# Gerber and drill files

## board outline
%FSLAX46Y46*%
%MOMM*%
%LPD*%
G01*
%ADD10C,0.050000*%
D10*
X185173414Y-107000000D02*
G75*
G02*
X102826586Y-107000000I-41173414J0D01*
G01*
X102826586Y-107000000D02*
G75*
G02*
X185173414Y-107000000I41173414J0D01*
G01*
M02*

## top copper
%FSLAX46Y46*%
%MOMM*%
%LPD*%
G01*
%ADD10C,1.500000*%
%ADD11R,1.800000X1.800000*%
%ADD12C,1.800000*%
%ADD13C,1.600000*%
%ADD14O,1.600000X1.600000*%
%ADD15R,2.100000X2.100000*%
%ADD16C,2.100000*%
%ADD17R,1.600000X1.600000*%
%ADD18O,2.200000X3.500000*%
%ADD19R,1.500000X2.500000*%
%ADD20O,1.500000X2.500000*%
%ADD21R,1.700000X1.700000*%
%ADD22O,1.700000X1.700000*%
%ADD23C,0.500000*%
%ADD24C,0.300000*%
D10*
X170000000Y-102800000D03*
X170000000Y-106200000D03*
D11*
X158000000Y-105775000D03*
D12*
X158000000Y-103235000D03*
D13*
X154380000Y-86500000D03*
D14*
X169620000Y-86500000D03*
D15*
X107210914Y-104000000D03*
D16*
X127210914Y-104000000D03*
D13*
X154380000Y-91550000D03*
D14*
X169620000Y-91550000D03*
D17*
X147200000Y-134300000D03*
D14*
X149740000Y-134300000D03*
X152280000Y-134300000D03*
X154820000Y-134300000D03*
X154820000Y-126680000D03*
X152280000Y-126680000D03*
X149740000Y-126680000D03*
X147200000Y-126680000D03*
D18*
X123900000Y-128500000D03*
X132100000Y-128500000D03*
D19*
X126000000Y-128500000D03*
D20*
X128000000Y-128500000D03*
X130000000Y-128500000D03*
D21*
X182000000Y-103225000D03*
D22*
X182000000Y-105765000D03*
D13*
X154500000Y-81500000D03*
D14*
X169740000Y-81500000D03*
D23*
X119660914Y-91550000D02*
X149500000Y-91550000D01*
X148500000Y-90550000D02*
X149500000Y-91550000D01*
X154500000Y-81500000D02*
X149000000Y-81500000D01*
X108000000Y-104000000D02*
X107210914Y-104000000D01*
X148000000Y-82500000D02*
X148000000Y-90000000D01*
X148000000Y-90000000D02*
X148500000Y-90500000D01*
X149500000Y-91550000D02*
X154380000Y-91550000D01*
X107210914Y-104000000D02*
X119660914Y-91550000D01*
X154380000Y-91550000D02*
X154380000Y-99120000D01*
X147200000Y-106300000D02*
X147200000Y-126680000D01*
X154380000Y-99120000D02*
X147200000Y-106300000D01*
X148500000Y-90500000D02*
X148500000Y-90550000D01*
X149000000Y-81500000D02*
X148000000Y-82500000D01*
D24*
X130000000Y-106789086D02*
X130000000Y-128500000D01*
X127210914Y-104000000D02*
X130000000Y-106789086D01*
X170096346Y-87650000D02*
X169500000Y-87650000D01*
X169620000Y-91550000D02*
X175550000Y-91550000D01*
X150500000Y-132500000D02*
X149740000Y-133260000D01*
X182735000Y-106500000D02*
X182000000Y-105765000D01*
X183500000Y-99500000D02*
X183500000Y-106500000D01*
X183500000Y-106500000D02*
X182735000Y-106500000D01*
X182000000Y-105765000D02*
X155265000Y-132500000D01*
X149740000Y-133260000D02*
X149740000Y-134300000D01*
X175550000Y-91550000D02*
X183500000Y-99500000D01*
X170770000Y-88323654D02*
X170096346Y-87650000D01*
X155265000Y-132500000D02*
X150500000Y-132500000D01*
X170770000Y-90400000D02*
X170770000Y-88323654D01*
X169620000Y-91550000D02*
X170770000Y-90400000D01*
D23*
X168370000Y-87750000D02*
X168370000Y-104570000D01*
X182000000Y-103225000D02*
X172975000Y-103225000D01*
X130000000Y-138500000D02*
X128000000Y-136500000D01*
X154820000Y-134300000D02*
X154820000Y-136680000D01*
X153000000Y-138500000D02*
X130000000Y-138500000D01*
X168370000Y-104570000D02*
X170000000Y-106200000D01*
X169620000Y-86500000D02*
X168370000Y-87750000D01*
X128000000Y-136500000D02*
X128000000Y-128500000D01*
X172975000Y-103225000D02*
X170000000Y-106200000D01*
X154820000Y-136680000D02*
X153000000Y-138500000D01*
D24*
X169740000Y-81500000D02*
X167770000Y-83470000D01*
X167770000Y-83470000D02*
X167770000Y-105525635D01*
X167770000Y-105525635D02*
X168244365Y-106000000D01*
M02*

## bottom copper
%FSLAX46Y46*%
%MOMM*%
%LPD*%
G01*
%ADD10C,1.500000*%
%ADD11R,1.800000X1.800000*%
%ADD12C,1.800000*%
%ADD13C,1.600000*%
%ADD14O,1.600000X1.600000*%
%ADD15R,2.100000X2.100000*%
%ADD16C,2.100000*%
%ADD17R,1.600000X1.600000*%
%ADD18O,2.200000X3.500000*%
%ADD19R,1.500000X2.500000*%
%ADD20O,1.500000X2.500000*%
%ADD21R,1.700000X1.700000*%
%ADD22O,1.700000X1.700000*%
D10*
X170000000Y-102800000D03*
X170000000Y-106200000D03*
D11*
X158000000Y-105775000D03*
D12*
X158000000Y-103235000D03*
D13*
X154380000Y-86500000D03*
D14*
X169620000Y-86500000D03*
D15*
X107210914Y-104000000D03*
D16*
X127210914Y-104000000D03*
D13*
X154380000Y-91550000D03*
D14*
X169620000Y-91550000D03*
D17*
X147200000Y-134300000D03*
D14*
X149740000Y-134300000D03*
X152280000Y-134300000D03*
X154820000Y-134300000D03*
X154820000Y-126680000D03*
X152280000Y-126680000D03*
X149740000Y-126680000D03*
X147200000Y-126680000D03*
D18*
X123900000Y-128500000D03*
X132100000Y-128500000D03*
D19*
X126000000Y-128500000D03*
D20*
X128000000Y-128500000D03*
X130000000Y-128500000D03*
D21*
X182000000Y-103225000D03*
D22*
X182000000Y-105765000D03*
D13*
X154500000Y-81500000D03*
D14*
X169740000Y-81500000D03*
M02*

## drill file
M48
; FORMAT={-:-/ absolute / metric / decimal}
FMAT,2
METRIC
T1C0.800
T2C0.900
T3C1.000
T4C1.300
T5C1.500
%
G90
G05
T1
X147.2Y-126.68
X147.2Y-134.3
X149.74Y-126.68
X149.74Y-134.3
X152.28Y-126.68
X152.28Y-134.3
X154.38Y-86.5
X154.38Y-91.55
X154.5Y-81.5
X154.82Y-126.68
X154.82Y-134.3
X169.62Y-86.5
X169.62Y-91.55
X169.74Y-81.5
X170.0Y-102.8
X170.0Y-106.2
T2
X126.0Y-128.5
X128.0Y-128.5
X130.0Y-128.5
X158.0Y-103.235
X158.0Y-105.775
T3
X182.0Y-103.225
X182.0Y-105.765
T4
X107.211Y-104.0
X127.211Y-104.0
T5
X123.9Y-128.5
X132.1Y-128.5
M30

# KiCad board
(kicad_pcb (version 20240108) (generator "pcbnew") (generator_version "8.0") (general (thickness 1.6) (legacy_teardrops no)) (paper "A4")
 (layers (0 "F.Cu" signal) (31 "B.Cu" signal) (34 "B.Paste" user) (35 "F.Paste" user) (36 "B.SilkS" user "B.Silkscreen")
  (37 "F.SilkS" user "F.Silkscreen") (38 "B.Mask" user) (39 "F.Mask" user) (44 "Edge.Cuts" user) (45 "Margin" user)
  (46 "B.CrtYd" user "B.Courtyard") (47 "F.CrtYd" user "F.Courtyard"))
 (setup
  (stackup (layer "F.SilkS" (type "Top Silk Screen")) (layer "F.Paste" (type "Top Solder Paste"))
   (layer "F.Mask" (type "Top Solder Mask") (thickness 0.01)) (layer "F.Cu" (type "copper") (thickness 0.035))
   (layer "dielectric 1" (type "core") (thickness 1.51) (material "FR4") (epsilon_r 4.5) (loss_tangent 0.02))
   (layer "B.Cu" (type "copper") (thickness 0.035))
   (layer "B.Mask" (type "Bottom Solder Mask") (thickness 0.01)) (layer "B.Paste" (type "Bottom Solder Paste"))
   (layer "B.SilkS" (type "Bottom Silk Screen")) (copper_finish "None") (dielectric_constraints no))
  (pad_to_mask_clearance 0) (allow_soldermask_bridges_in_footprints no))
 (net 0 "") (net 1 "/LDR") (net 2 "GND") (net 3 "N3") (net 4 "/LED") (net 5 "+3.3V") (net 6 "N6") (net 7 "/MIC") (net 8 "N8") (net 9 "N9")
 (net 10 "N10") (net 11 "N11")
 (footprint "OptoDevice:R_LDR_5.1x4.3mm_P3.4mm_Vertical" (layer "F.Cu") (at 170 102.8 -90)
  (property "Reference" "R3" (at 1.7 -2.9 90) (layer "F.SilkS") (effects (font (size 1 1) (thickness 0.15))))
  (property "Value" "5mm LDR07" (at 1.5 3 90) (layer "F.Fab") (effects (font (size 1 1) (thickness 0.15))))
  (pad "1" thru_hole circle (at 0 0 270) (size 1.5 1.5) (drill 0.8) (layers "*.Cu" "*.Mask") (remove_unused_layers no) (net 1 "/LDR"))
  (pad "2" thru_hole circle (at 3.4 0 270) (size 1.5 1.5) (drill 0.8) (layers "*.Cu" "*.Mask") (remove_unused_layers no) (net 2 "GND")))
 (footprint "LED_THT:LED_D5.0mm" (layer "F.Cu") (at 158 105.775 90)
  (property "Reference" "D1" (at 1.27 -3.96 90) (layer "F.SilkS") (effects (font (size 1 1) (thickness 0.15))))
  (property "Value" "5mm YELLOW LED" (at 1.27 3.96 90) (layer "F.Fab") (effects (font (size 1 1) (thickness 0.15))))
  (pad "1" thru_hole rect (at 0 0 90) (size 1.8 1.8) (drill 0.9) (layers "*.Cu" "*.Mask") (remove_unused_layers no) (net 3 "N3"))
  (pad "2" thru_hole circle (at 2.54 0 90) (size 1.8 1.8) (drill 0.9) (layers "*.Cu" "*.Mask") (remove_unused_layers no) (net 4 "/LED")))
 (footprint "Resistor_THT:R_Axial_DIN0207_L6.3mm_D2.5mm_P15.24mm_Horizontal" (layer "F.Cu") (at 154.38 86.5)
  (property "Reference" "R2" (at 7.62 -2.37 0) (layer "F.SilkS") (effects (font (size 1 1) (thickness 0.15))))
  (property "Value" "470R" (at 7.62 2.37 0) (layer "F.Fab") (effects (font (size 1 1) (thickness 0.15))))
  (pad "1" thru_hole circle (at 0 0) (size 1.6 1.6) (drill 0.8) (layers "*.Cu" "*.Mask") (remove_unused_layers no) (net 3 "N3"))
  (pad "2" thru_hole oval (at 15.24 0) (size 1.6 1.6) (drill 0.8) (layers "*.Cu" "*.Mask") (remove_unused_layers no) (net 2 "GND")))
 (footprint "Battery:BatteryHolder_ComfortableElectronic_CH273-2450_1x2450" (layer "F.Cu") (at 107.210914 104)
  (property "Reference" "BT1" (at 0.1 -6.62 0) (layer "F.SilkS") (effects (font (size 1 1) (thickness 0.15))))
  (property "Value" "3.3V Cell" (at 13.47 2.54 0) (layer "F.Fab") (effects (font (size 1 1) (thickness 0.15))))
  (pad "1" thru_hole rect (at 0 0 270) (size 2.1 2.1) (drill 1.3) (layers "*.Cu" "*.Mask") (remove_unused_layers no) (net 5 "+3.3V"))
  (pad "2" thru_hole circle (at 20 0 270) (size 2.1 2.1) (drill 1.3) (layers "*.Cu" "*.Mask") (remove_unused_layers no) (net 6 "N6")))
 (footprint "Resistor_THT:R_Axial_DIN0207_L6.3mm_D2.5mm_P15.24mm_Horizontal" (layer "F.Cu") (at 154.38 91.55)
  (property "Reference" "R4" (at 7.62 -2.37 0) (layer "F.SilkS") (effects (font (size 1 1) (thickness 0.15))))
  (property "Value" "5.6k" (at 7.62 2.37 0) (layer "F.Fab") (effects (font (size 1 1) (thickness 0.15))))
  (pad "1" thru_hole circle (at 0 0) (size 1.6 1.6) (drill 0.8) (layers "*.Cu" "*.Mask") (remove_unused_layers no) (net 5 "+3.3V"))
  (pad "2" thru_hole oval (at 15.24 0) (size 1.6 1.6) (drill 0.8) (layers "*.Cu" "*.Mask") (remove_unused_layers no) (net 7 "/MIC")))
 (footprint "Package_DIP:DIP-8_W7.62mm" (layer "F.Cu") (at 147.2 134.3 90)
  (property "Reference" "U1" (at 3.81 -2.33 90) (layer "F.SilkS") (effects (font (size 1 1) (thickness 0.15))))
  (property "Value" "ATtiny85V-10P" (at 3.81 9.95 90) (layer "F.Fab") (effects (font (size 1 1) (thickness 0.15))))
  (pad "1" thru_hole rect (at 0 0 90) (size 1.6 1.6) (drill 0.8) (layers "*.Cu" "*.Mask") (remove_unused_layers no) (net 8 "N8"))
  (pad "2" thru_hole oval (at 0 2.54 90) (size 1.6 1.6) (drill 0.8) (layers "*.Cu" "*.Mask") (remove_unused_layers no) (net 7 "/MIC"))
  (pad "3" thru_hole oval (at 0 5.08 90) (size 1.6 1.6) (drill 0.8) (layers "*.Cu" "*.Mask") (remove_unused_layers no) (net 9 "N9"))
  (pad "4" thru_hole oval (at 0 7.62 90) (size 1.6 1.6) (drill 0.8) (layers "*.Cu" "*.Mask") (remove_unused_layers no) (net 2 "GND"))
  (pad "5" thru_hole oval (at 7.62 7.62 90) (size 1.6 1.6) (drill 0.8) (layers "*.Cu" "*.Mask") (remove_unused_layers no) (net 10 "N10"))
  (pad "6" thru_hole oval (at 7.62 5.08 90) (size 1.6 1.6) (drill 0.8) (layers "*.Cu" "*.Mask") (remove_unused_layers no) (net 4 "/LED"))
  (pad "7" thru_hole oval (at 7.62 2.54 90) (size 1.6 1.6) (drill 0.8) (layers "*.Cu" "*.Mask") (remove_unused_layers no) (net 1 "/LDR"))
  (pad "8" thru_hole oval (at 7.62 0 90) (size 1.6 1.6) (drill 0.8) (layers "*.Cu" "*.Mask") (remove_unused_layers no) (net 5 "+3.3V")))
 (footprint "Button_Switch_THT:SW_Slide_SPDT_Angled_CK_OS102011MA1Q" (layer "F.Cu") (at 126 128.5)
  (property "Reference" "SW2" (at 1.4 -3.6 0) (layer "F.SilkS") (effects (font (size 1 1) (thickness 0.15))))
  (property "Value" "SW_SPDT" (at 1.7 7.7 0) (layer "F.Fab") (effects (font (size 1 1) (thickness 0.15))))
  (pad "" thru_hole oval (at -2.1 0) (size 2.2 3.5) (drill 1.5) (layers "*.Cu" "*.Mask") (remove_unused_layers no))
  (pad "" thru_hole oval (at 6.1 0) (size 2.2 3.5) (drill 1.5) (layers "*.Cu" "*.Mask") (remove_unused_layers no))
  (pad "1" thru_hole rect (at 0 0) (size 1.5 2.5) (drill 0.9) (layers "*.Cu" "*.Mask") (remove_unused_layers no) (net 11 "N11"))
  (pad "2" thru_hole oval (at 2 0) (size 1.5 2.5) (drill 0.9) (layers "*.Cu" "*.Mask") (remove_unused_layers no) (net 2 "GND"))
  (pad "3" thru_hole oval (at 4 0) (size 1.5 2.5) (drill 0.9) (layers "*.Cu" "*.Mask") (remove_unused_layers no) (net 6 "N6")))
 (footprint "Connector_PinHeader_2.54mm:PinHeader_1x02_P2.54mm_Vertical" (layer "F.Cu") (at 182 103.225)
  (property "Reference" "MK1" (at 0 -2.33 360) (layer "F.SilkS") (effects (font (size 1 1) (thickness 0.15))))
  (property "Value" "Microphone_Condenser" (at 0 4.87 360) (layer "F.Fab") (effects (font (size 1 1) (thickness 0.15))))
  (pad "1" thru_hole rect (at 0 0) (size 1.7 1.7) (drill 1) (layers "*.Cu" "*.Mask") (remove_unused_layers no) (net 2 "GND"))
  (pad "2" thru_hole oval (at 0 2.54) (size 1.7 1.7) (drill 1) (layers "*.Cu" "*.Mask") (remove_unused_layers no) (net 7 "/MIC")))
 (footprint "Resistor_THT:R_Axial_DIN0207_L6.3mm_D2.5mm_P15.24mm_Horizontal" (layer "F.Cu") (at 154.5 81.5)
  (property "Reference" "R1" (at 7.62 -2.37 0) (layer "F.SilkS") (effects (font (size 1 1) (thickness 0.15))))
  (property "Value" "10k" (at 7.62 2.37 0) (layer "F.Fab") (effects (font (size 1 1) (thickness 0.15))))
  (pad "1" thru_hole circle (at 0 0) (size 1.6 1.6) (drill 0.8) (layers "*.Cu" "*.Mask") (remove_unused_layers no) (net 5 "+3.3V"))
  (pad "2" thru_hole oval (at 15.24 0) (size 1.6 1.6) (drill 0.8) (layers "*.Cu" "*.Mask") (remove_unused_layers no) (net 1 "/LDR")))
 (gr_circle (center 144 107) (end 106.5 90) (stroke (width 0.05) (type default)) (fill none) (layer "Edge.Cuts"))
 (segment (start 119.660914 91.55) (end 149.5 91.55) (width 0.5) (layer "F.Cu") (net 5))
 (segment (start 148.5 90.55) (end 149.5 91.55) (width 0.5) (layer "F.Cu") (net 5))
 (segment (start 154.5 81.5) (end 149 81.5) (width 0.5) (layer "F.Cu") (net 5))
 (segment (start 108 104) (end 107.210914 104) (width 0.5) (layer "F.Cu") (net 5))
 (segment (start 148 82.5) (end 148 90) (width 0.5) (layer "F.Cu") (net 5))
 (segment (start 148 90) (end 148.5 90.5) (width 0.5) (layer "F.Cu") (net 5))
 (segment (start 149.5 91.55) (end 154.38 91.55) (width 0.5) (layer "F.Cu") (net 5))
 (segment (start 107.210914 104) (end 119.660914 91.55) (width 0.5) (layer "F.Cu") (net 5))
 (segment (start 154.38 91.55) (end 154.38 99.12) (width 0.5) (layer "F.Cu") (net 5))
 (segment (start 147.2 106.3) (end 147.2 126.68) (width 0.5) (layer "F.Cu") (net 5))
 (segment (start 154.38 99.12) (end 147.2 106.3) (width 0.5) (layer "F.Cu") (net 5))
 (segment (start 148.5 90.5) (end 148.5 90.55) (width 0.5) (layer "F.Cu") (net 5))
 (segment (start 149 81.5) (end 148 82.5) (width 0.5) (layer "F.Cu") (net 5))
 (segment (start 130 106.789086) (end 130 128.5) (width 0.3) (layer "F.Cu") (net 6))
 (segment (start 127.210914 104) (end 130 106.789086) (width 0.3) (layer "F.Cu") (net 6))
 (segment (start 170.096346 87.65) (end 169.5 87.65) (width 0.3) (layer "F.Cu") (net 7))
 (segment (start 169.62 91.55) (end 175.55 91.55) (width 0.3) (layer "F.Cu") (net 7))
 (segment (start 150.5 132.5) (end 149.74 133.26) (width 0.3) (layer "F.Cu") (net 7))
 (segment (start 182.735 106.5) (end 182 105.765) (width 0.3) (layer "F.Cu") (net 7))
 (segment (start 183.5 99.5) (end 183.5 106.5) (width 0.3) (layer "F.Cu") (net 7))
 (segment (start 183.5 106.5) (end 182.735 106.5) (width 0.3) (layer "F.Cu") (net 7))
 (segment (start 182 105.765) (end 155.265 132.5) (width 0.3) (layer "F.Cu") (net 7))
 (segment (start 149.74 133.26) (end 149.74 134.3) (width 0.3) (layer "F.Cu") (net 7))
 (segment (start 175.55 91.55) (end 183.5 99.5) (width 0.3) (layer "F.Cu") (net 7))
 (segment (start 170.77 88.323654) (end 170.096346 87.65) (width 0.3) (layer "F.Cu") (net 7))
 (segment (start 155.265 132.5) (end 150.5 132.5) (width 0.3) (layer "F.Cu") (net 7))
 (segment (start 170.77 90.4) (end 170.77 88.323654) (width 0.3) (layer "F.Cu") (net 7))
 (segment (start 169.62 91.55) (end 170.77 90.4) (width 0.3) (layer "F.Cu") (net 7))
 (segment (start 168.37 87.75) (end 168.37 104.57) (width 0.5) (layer "F.Cu") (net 2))
 (segment (start 182 103.225) (end 172.975 103.225) (width 0.5) (layer "F.Cu") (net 2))
 (segment (start 130 138.5) (end 128 136.5) (width 0.5) (layer "F.Cu") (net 2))
 (segment (start 154.82 134.3) (end 154.82 136.68) (width 0.5) (layer "F.Cu") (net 2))
 (segment (start 153 138.5) (end 130 138.5) (width 0.5) (layer "F.Cu") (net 2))
 (segment (start 168.37 104.57) (end 170 106.2) (width 0.5) (layer "F.Cu") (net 2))
 (segment (start 169.62 86.5) (end 168.37 87.75) (width 0.5) (layer "F.Cu") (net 2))
 (segment (start 128 136.5) (end 128 128.5) (width 0.5) (layer "F.Cu") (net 2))
 (segment (start 172.975 103.225) (end 170 106.2) (width 0.5) (layer "F.Cu") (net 2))
 (segment (start 154.82 136.68) (end 153 138.5) (width 0.5) (layer "F.Cu") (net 2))
 (segment (start 169.74 81.5) (end 167.77 83.47) (width 0.3) (layer "F.Cu") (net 1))
 (segment (start 167.77 83.47) (end 167.77 105.525635) (width 0.3) (layer "F.Cu") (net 1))
 (segment (start 167.77 105.525635) (end 168.244365 106) (width 0.3) (layer "F.Cu") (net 1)))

